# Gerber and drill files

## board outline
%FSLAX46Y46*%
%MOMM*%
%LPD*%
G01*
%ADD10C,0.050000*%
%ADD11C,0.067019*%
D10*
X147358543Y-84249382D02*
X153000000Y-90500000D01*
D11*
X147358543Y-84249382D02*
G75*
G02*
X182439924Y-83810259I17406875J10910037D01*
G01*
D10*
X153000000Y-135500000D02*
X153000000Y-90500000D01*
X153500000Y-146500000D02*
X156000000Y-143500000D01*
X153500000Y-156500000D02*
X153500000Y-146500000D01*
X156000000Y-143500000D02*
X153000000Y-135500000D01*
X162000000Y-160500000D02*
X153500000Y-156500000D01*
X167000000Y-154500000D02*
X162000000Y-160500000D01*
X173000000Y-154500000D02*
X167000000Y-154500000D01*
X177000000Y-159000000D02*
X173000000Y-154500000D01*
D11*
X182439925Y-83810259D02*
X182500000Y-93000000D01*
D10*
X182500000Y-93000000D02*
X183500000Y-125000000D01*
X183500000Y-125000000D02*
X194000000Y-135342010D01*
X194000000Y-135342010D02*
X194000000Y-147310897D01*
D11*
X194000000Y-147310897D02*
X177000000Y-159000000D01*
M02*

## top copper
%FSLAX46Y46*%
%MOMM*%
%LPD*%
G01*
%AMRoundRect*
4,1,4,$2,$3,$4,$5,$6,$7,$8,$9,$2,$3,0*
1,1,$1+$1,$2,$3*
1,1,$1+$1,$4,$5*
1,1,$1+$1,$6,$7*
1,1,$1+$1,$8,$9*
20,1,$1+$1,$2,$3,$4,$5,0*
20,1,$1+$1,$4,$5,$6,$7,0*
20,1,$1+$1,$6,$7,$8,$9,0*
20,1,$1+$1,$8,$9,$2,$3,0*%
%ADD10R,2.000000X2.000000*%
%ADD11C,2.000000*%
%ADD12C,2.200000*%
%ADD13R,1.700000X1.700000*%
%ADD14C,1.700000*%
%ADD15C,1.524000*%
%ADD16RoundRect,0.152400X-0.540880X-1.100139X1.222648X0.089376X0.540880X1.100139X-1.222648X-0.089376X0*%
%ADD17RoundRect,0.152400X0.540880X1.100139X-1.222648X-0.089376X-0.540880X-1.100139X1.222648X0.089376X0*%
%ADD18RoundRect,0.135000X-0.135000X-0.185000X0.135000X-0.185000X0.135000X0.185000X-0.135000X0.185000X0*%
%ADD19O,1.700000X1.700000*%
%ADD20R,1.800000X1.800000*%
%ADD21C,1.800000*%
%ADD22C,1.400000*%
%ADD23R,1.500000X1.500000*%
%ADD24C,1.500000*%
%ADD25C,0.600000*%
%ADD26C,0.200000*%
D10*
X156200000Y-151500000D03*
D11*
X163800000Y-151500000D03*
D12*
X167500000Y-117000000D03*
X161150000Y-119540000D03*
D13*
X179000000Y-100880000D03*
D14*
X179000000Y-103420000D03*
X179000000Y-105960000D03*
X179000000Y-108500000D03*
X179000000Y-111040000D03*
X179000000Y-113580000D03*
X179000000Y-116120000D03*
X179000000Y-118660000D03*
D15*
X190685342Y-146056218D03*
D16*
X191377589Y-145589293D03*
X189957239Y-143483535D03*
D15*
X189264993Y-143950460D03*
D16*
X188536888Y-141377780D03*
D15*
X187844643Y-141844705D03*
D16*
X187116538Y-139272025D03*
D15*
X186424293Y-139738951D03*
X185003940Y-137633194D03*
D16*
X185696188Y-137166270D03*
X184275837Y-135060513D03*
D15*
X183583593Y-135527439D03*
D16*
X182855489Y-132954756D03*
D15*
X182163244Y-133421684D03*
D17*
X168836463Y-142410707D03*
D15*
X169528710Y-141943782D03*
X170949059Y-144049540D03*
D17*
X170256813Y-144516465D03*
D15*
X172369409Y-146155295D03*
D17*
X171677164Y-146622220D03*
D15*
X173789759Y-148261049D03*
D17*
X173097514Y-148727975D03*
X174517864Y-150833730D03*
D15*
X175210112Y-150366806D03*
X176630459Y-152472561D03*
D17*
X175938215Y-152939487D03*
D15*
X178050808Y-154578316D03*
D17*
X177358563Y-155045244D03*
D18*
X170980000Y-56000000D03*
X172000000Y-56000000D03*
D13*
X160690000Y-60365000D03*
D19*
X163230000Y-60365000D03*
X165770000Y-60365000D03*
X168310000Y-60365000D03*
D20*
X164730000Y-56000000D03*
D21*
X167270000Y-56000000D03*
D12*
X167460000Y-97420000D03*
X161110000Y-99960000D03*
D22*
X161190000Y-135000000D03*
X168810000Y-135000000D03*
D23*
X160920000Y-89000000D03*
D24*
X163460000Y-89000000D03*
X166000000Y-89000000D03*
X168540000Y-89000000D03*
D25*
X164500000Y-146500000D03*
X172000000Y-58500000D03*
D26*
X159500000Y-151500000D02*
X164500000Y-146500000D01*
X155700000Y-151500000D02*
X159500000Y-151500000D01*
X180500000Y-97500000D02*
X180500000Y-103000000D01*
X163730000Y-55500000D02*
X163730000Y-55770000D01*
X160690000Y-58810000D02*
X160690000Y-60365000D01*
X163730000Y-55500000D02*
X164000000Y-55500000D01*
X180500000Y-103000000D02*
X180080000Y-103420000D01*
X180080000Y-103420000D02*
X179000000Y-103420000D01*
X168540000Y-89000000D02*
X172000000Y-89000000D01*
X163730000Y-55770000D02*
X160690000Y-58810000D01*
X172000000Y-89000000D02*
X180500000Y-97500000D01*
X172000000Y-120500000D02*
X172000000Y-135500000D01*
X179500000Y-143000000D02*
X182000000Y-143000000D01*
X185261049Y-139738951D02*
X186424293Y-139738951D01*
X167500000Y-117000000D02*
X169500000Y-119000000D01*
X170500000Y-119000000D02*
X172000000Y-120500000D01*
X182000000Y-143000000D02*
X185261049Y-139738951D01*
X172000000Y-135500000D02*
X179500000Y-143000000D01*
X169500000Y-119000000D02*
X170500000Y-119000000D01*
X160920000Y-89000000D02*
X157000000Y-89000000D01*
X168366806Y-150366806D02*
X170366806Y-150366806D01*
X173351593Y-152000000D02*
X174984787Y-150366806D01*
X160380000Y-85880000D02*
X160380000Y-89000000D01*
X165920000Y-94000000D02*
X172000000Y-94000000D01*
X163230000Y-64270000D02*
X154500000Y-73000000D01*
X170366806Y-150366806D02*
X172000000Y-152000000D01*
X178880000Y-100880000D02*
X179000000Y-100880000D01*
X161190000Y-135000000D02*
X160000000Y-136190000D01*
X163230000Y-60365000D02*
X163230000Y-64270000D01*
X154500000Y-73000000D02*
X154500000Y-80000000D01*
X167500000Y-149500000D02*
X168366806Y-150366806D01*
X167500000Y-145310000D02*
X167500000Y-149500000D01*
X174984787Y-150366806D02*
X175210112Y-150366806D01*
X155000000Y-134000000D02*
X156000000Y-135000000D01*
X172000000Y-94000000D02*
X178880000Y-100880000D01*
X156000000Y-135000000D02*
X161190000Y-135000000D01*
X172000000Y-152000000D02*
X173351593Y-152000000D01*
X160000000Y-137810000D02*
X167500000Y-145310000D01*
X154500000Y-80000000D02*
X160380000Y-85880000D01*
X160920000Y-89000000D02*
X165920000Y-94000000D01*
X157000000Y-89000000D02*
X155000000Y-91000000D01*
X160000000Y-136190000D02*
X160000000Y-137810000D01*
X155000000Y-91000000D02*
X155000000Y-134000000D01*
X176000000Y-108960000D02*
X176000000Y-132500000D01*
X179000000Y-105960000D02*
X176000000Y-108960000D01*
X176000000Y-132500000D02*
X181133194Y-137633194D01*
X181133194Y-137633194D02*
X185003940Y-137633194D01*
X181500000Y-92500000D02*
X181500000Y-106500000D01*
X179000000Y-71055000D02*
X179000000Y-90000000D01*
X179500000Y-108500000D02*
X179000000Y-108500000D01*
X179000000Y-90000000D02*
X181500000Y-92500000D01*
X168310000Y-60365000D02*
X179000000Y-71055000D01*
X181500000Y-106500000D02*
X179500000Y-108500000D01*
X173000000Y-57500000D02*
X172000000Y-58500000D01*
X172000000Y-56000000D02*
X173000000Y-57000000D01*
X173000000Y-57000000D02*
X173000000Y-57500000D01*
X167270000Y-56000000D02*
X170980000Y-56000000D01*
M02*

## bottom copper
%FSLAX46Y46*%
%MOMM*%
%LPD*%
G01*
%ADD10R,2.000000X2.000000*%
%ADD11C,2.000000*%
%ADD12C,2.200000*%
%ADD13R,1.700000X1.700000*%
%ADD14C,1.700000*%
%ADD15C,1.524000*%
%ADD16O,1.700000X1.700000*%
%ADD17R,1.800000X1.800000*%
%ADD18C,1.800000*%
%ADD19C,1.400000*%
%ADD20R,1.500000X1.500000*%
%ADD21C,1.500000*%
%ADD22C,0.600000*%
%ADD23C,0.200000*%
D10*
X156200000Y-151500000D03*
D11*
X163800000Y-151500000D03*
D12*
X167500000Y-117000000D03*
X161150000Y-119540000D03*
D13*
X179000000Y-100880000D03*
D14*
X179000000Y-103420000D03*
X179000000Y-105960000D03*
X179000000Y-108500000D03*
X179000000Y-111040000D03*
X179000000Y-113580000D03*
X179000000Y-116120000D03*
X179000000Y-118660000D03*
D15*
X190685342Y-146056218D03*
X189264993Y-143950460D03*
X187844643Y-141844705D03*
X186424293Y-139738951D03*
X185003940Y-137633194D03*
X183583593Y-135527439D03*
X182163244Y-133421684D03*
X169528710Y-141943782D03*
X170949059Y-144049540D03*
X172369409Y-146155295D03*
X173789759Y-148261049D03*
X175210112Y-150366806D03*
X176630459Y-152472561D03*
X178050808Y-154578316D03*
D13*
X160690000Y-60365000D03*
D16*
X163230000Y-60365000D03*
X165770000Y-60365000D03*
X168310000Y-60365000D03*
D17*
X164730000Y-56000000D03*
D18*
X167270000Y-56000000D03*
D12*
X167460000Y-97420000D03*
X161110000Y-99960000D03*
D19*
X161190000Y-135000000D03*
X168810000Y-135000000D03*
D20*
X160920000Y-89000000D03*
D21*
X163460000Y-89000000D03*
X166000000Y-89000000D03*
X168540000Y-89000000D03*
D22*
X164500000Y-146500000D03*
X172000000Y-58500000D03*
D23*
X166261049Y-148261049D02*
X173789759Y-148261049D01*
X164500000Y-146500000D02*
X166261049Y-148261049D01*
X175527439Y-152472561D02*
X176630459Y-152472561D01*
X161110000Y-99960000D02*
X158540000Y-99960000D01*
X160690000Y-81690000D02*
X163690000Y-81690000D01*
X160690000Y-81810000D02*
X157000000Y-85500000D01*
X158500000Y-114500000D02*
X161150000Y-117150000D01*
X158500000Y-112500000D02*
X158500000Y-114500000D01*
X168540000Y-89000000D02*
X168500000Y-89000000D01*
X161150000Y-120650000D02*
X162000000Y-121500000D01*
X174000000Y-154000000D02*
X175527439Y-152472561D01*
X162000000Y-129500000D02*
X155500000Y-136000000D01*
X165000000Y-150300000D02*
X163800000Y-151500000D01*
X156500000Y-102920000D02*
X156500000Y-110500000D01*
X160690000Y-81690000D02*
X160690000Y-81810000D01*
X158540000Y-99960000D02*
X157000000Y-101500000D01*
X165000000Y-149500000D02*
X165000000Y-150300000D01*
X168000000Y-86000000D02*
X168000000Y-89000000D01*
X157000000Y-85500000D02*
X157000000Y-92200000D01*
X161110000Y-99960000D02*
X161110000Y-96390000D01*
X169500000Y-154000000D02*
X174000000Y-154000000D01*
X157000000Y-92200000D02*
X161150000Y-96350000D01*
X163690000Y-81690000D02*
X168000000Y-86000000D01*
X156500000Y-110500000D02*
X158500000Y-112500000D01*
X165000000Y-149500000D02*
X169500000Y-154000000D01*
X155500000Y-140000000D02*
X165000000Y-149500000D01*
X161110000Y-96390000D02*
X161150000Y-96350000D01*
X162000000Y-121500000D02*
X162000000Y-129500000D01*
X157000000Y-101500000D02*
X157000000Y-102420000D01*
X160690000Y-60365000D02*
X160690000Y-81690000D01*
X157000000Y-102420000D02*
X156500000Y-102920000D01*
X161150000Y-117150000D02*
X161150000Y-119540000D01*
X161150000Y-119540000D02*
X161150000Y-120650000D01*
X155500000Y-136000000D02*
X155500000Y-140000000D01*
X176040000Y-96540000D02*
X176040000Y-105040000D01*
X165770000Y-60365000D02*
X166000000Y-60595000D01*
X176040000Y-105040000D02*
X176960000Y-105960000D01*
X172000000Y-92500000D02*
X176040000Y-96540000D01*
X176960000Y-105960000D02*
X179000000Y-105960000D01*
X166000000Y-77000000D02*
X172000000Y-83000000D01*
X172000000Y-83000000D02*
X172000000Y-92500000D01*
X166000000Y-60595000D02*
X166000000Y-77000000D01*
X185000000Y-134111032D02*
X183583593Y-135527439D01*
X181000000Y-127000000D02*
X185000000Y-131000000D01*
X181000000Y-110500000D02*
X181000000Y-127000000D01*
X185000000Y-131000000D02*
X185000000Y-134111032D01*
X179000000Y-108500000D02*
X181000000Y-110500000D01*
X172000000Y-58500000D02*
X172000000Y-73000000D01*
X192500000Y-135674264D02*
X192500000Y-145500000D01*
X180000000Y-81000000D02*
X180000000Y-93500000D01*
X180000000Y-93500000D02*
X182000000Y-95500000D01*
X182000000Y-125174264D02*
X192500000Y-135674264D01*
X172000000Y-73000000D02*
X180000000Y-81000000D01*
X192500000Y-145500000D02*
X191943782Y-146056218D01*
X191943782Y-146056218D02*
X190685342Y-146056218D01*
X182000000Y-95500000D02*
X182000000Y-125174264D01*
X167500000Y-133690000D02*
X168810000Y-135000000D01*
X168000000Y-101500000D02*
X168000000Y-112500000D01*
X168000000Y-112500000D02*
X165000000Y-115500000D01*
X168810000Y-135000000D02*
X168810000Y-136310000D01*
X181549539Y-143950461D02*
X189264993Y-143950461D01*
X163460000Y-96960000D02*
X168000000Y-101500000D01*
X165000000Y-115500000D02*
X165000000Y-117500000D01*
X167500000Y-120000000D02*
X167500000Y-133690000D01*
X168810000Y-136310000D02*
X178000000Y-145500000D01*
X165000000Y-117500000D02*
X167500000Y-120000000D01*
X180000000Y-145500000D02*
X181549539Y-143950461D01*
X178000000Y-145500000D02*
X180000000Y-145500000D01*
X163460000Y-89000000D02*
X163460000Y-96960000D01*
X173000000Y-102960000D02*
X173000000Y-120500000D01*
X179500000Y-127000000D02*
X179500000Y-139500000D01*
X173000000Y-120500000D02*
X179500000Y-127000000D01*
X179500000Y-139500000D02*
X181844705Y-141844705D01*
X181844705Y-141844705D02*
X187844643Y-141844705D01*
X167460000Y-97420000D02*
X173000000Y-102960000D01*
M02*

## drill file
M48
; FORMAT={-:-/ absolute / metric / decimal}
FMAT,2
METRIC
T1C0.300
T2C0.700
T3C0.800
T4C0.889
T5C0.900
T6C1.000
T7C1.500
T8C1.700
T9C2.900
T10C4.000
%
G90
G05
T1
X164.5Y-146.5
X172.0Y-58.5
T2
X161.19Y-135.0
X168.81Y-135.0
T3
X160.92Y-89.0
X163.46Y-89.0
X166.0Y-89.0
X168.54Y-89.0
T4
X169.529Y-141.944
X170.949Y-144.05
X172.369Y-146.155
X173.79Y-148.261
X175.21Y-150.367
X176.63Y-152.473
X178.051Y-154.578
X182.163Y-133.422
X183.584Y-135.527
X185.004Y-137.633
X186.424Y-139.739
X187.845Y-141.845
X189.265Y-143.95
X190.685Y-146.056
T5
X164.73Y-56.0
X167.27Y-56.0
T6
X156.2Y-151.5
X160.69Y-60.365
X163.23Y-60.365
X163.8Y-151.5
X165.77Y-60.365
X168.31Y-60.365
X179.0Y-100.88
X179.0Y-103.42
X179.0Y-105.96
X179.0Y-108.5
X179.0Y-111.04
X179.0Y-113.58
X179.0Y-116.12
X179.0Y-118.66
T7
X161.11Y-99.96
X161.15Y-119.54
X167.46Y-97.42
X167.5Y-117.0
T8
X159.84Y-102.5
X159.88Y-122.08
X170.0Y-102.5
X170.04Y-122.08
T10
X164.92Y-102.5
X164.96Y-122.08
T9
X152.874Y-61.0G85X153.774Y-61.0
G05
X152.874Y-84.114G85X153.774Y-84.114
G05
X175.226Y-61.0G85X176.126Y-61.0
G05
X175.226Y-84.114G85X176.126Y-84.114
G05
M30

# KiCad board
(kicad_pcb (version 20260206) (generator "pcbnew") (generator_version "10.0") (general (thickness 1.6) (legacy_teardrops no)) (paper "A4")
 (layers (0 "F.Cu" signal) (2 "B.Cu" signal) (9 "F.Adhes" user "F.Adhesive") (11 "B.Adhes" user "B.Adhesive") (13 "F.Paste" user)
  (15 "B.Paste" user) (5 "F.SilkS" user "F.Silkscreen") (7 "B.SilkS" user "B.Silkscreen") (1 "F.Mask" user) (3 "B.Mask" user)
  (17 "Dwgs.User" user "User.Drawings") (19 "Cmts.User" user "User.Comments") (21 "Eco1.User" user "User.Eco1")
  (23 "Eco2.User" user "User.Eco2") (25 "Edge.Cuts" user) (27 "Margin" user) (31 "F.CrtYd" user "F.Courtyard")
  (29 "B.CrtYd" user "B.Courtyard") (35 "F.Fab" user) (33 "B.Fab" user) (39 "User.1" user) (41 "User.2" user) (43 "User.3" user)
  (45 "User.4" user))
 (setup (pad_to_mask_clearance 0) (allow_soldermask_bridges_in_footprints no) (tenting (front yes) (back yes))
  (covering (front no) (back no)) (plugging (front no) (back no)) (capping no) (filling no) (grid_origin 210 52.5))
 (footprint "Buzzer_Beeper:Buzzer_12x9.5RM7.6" (layer "F.Cu") (at 156.2 151.5)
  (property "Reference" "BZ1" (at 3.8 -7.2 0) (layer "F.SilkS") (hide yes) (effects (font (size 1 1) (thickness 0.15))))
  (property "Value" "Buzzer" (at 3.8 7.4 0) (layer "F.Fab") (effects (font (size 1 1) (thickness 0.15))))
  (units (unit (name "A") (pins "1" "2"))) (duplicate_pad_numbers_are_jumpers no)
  (pad "1" thru_hole rect (at 0 0) (size 2 2) (drill 1) (layers "*.Cu" "*.Mask") (remove_unused_layers no) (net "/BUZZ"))
  (pad "2" thru_hole circle (at 7.6 0) (size 2 2) (drill 1) (layers "*.Cu" "*.Mask") (remove_unused_layers no) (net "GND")))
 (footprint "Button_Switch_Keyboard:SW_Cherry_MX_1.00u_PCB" (layer "F.Cu") (at 167.5 117)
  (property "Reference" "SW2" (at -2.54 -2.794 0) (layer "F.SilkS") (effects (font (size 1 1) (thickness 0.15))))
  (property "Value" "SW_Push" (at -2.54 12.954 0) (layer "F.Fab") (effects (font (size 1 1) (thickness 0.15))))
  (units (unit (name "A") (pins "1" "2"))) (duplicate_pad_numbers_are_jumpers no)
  (pad "" np_thru_hole circle (at -7.62 5.08) (size 1.7 1.7) (drill 1.7) (layers "*.Cu" "*.Mask"))
  (pad "" np_thru_hole circle (at -2.54 5.08) (size 4 4) (drill 4) (layers "*.Cu" "*.Mask"))
  (pad "" np_thru_hole circle (at 2.54 5.08) (size 1.7 1.7) (drill 1.7) (layers "*.Cu" "*.Mask"))
  (pad "1" thru_hole circle (at 0 0) (size 2.2 2.2) (drill 1.5) (layers "*.Cu" "*.Mask") (remove_unused_layers no) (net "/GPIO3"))
  (pad "2" thru_hole circle (at -6.35 2.54) (size 2.2 2.2) (drill 1.5) (layers "*.Cu" "*.Mask") (remove_unused_layers no) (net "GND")))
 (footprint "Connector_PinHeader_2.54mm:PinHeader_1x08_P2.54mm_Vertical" (layer "F.Cu") (at 179 100.88)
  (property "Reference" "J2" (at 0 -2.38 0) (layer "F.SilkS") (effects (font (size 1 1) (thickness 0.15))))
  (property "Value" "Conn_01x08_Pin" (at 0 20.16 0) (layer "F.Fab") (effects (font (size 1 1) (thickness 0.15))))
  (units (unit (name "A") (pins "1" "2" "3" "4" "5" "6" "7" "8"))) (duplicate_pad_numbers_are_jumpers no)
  (pad "1" thru_hole rect (at 0 0) (size 1.7 1.7) (drill 1) (layers "*.Cu" "*.Mask") (remove_unused_layers no) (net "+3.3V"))
  (pad "2" thru_hole circle (at 0 2.54) (size 1.7 1.7) (drill 1) (layers "*.Cu" "*.Mask") (remove_unused_layers no) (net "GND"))
  (pad "3" thru_hole circle (at 0 5.08) (size 1.7 1.7) (drill 1) (layers "*.Cu" "*.Mask") (remove_unused_layers no) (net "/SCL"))
  (pad "4" thru_hole circle (at 0 7.62) (size 1.7 1.7) (drill 1) (layers "*.Cu" "*.Mask") (remove_unused_layers no) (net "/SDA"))
  (pad "5" thru_hole circle (at 0 10.16) (size 1.7 1.7) (drill 1) (layers "*.Cu" "*.Mask") (remove_unused_layers no)
   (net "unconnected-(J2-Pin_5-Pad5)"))
  (pad "6" thru_hole circle (at 0 12.7) (size 1.7 1.7) (drill 1) (layers "*.Cu" "*.Mask") (remove_unused_layers no)
   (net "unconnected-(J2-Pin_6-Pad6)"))
  (pad "7" thru_hole circle (at 0 15.24) (size 1.7 1.7) (drill 1) (layers "*.Cu" "*.Mask") (remove_unused_layers no)
   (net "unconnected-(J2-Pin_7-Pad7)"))
  (pad "8" thru_hole circle (at 0 17.78) (size 1.7 1.7) (drill 1) (layers "*.Cu" "*.Mask") (remove_unused_layers no)
   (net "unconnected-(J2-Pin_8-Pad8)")))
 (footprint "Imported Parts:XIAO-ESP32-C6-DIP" (layer "F.Cu") (at 180.107026 144 -56)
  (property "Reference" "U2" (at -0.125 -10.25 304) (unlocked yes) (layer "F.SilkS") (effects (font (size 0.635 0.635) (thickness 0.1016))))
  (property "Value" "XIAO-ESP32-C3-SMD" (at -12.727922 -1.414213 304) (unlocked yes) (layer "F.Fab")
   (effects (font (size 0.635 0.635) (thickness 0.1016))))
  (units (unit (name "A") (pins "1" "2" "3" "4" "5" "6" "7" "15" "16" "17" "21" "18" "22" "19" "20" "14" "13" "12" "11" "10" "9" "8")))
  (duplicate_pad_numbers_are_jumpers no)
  (pad "1" thru_hole circle (at 7.620001 -7.619999 34) (size 1.524 1.524) (drill 0.889) (layers "*.Cu" "*.Mask") (remove_unused_layers no)
   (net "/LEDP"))
  (pad "1" smd roundrect (at 7.620002 -8.454999 34) (size 2.432 1.524) (layers "F.Cu" "F.Mask") (roundrect_rratio 0.1) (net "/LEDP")
   (thermal_bridge_angle 45))
  (pad "2" smd roundrect (at 5.08 -8.455 34) (size 2.432 1.524) (layers "F.Cu" "F.Mask") (roundrect_rratio 0.1) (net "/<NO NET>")
   (thermal_bridge_angle 45))
  (pad "2" thru_hole circle (at 5.08 -7.620001 34) (size 1.524 1.524) (drill 0.889) (layers "*.Cu" "*.Mask") (remove_unused_layers no)
   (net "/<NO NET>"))
  (pad "3" smd roundrect (at 2.54 -8.454999 34) (size 2.432 1.524) (layers "F.Cu" "F.Mask") (roundrect_rratio 0.1) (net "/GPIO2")
   (thermal_bridge_angle 45))
  (pad "3" thru_hole circle (at 2.54 -7.620001 34) (size 1.524 1.524) (drill 0.889) (layers "*.Cu" "*.Mask") (remove_unused_layers no)
   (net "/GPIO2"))
  (pad "4" smd roundrect (at 0 -8.454999 34) (size 2.432 1.524) (layers "F.Cu" "F.Mask") (roundrect_rratio 0.1) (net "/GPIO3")
   (thermal_bridge_angle 45))
  (pad "4" thru_hole circle (at 0.000001 -7.62 34) (size 1.524 1.524) (drill 0.889) (layers "*.Cu" "*.Mask") (remove_unused_layers no)
   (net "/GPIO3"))
  (pad "5" thru_hole circle (at -2.540002 -7.619998 34) (size 1.524 1.524) (drill 0.889) (layers "*.Cu" "*.Mask") (remove_unused_layers no)
   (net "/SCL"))
  (pad "5" smd roundrect (at -2.539999 -8.454999 34) (size 2.432 1.524) (layers "F.Cu" "F.Mask") (roundrect_rratio 0.1) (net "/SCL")
   (thermal_bridge_angle 45))
  (pad "6" smd roundrect (at -5.080001 -8.454999 34) (size 2.432 1.524) (layers "F.Cu" "F.Mask") (roundrect_rratio 0.1) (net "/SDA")
   (thermal_bridge_angle 45))
  (pad "6" thru_hole circle (at -5.08 -7.620001 34) (size 1.524 1.524) (drill 0.889) (layers "*.Cu" "*.Mask") (remove_unused_layers no)
   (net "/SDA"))
  (pad "7" smd roundrect (at -7.620001 -8.455001 34) (size 2.432 1.524) (layers "F.Cu" "F.Mask") (roundrect_rratio 0.1)
   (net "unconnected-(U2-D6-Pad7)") (thermal_bridge_angle 45))
  (pad "7" thru_hole circle (at -7.619999 -7.620001 34) (size 1.524 1.524) (drill 0.889) (layers "*.Cu" "*.Mask") (remove_unused_layers no)
   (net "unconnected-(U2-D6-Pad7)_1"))
  (pad "8" smd roundrect (at -7.620002 8.454999 214) (size 2.432 1.524) (layers "F.Cu" "F.Mask") (roundrect_rratio 0.1)
   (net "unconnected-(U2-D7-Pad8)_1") (thermal_bridge_angle 45))
  (pad "8" thru_hole circle (at -7.620001 7.619999 214) (size 1.524 1.524) (drill 0.889) (layers "*.Cu" "*.Mask") (remove_unused_layers no)
   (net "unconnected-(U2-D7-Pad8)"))
  (pad "9" thru_hole circle (at -5.08 7.620001 214) (size 1.524 1.524) (drill 0.889) (layers "*.Cu" "*.Mask") (remove_unused_layers no)
   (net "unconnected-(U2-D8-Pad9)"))
  (pad "9" smd roundrect (at -5.08 8.455 214) (size 2.432 1.524) (layers "F.Cu" "F.Mask") (roundrect_rratio 0.1)
   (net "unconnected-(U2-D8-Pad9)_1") (thermal_bridge_angle 45))
  (pad "10" thru_hole circle (at -2.54 7.620001 214) (size 1.524 1.524) (drill 0.889) (layers "*.Cu" "*.Mask") (remove_unused_layers no)
   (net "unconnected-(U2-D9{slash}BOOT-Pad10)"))
  (pad "10" smd roundrect (at -2.54 8.454999 214) (size 2.432 1.524) (layers "F.Cu" "F.Mask") (roundrect_rratio 0.1)
   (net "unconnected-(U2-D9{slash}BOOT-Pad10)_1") (thermal_bridge_angle 45))
  (pad "11" thru_hole circle (at -0.000001 7.62 214) (size 1.524 1.524) (drill 0.889) (layers "*.Cu" "*.Mask") (remove_unused_layers no)
   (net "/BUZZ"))
  (pad "11" smd roundrect (at 0 8.454999 214) (size 2.432 1.524) (layers "F.Cu" "F.Mask") (roundrect_rratio 0.1) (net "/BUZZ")
   (thermal_bridge_angle 45))
  (pad "12" smd roundrect (at 2.539999 8.454999 214) (size 2.432 1.524) (layers "F.Cu" "F.Mask") (roundrect_rratio 0.1) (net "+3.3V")
   (thermal_bridge_angle 45))
  (pad "12" thru_hole circle (at 2.540002 7.619998 214) (size 1.524 1.524) (drill 0.889) (layers "*.Cu" "*.Mask") (remove_unused_layers no)
   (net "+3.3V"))
  (pad "13" thru_hole circle (at 5.08 7.620001 214) (size 1.524 1.524) (drill 0.889) (layers "*.Cu" "*.Mask") (remove_unused_layers no)
   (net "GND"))
  (pad "13" smd roundrect (at 5.080001 8.454999 214) (size 2.432 1.524) (layers "F.Cu" "F.Mask") (roundrect_rratio 0.1) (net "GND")
   (thermal_bridge_angle 45))
  (pad "14" thru_hole circle (at 7.619999 7.620001 214) (size 1.524 1.524) (drill 0.889) (layers "*.Cu" "*.Mask") (remove_unused_layers no)
   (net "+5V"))
  (pad "14" smd roundrect (at 7.620001 8.455001 214) (size 2.432 1.524) (layers "F.Cu" "F.Mask") (roundrect_rratio 0.1) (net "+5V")
   (thermal_bridge_angle 45)))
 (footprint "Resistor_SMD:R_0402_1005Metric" (layer "F.Cu") (at 171.49 56)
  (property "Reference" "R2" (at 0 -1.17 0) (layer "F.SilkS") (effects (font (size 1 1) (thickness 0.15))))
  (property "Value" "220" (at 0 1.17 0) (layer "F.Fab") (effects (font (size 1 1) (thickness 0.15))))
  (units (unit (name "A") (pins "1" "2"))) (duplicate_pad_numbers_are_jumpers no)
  (pad "1" smd roundrect (at -0.51 0) (size 0.54 0.64) (layers "F.Cu" "F.Mask" "F.Paste") (roundrect_rratio 0.25) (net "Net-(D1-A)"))
  (pad "2" smd roundrect (at 0.51 0) (size 0.54 0.64) (layers "F.Cu" "F.Mask" "F.Paste") (roundrect_rratio 0.25) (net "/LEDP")))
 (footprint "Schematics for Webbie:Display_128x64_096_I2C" (layer "F.Cu") (at 164.5 60.365)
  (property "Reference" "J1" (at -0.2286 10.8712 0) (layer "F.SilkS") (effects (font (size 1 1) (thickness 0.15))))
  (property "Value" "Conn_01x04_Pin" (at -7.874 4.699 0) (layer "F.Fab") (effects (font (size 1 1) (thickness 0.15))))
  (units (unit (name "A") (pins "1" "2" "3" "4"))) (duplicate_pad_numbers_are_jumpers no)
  (pad "" np_thru_hole oval (at -11.176 0.635) (size 3.8 2.9) (drill oval 3.8 2.9) (layers "*.Cu" "*.Mask"))
  (pad "" np_thru_hole oval (at -11.176 23.749) (size 3.8 2.9) (drill oval 3.8 2.9) (layers "*.Cu" "*.Mask"))
  (pad "" np_thru_hole oval (at 11.176 0.635) (size 3.8 2.9) (drill oval 3.8 2.9) (layers "*.Cu" "*.Mask"))
  (pad "" np_thru_hole oval (at 11.176 23.749) (size 3.8 2.9) (drill oval 3.8 2.9) (layers "*.Cu" "*.Mask"))
  (pad "1" thru_hole rect (at -3.81 0 90) (size 1.7 1.7) (drill 1) (layers "*.Cu" "*.Mask") (remove_unused_layers no) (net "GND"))
  (pad "2" thru_hole oval (at -1.27 0 90) (size 1.7 1.7) (drill 1) (layers "*.Cu" "*.Mask") (remove_unused_layers no) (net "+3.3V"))
  (pad "3" thru_hole oval (at 1.27 0 90) (size 1.7 1.7) (drill 1) (layers "*.Cu" "*.Mask") (remove_unused_layers no) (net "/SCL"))
  (pad "4" thru_hole oval (at 3.81 0 90) (size 1.7 1.7) (drill 1) (layers "*.Cu" "*.Mask") (remove_unused_layers no) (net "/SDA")))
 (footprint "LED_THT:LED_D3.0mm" (layer "F.Cu") (at 164.73 56)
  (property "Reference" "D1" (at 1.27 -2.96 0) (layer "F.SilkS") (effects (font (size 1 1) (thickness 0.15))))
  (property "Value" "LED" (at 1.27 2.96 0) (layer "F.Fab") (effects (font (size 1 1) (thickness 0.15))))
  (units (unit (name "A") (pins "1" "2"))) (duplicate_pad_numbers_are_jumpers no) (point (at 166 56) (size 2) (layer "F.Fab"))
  (pad "1" thru_hole rect (at 0 0) (size 1.8 1.8) (drill 0.9) (layers "*.Cu" "*.Mask") (remove_unused_layers no) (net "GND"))
  (pad "2" thru_hole circle (at 2.54 0) (size 1.8 1.8) (drill 0.9) (layers "*.Cu" "*.Mask") (remove_unused_layers no) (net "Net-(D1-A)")))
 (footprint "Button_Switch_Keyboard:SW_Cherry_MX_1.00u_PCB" (layer "F.Cu") (at 167.46 97.42)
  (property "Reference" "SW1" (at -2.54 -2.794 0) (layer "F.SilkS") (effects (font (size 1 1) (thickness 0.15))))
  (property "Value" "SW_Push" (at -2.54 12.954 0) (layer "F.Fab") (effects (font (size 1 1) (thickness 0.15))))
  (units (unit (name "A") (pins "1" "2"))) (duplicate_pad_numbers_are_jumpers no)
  (pad "" np_thru_hole circle (at -7.62 5.08) (size 1.7 1.7) (drill 1.7) (layers "*.Cu" "*.Mask"))
  (pad "" np_thru_hole circle (at -2.54 5.08) (size 4 4) (drill 4) (layers "*.Cu" "*.Mask"))
  (pad "" np_thru_hole circle (at 2.54 5.08) (size 1.7 1.7) (drill 1.7) (layers "*.Cu" "*.Mask"))
  (pad "1" thru_hole circle (at 0 0) (size 2.2 2.2) (drill 1.5) (layers "*.Cu" "*.Mask") (remove_unused_layers no) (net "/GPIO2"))
  (pad "2" thru_hole circle (at -6.35 2.54) (size 2.2 2.2) (drill 1.5) (layers "*.Cu" "*.Mask") (remove_unused_layers no) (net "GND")))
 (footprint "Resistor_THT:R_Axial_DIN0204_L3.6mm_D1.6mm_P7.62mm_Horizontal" (layer "F.Cu") (at 161.19 135)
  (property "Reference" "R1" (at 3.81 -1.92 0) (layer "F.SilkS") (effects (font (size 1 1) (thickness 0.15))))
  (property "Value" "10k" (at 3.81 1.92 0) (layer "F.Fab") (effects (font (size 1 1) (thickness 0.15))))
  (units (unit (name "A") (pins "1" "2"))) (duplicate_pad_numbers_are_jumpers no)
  (pad "1" thru_hole circle (at 0 0) (size 1.4 1.4) (drill 0.7) (layers "*.Cu" "*.Mask") (remove_unused_layers no) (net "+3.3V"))
  (pad "2" thru_hole circle (at 7.62 0) (size 1.4 1.4) (drill 0.7) (layers "*.Cu" "*.Mask") (remove_unused_layers no) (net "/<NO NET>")))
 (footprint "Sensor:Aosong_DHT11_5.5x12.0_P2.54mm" (layer "F.Cu") (at 160.92 89 90)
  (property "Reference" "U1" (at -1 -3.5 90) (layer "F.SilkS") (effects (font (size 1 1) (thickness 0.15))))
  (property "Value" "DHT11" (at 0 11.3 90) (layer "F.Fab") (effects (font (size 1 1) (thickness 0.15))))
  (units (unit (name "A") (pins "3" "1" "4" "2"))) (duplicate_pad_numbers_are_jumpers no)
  (pad "1" thru_hole rect (at 0 0 90) (size 1.5 1.5) (drill 0.8) (layers "*.Cu" "*.Mask") (remove_unused_layers no) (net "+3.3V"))
  (pad "2" thru_hole circle (at 0 2.54 90) (size 1.5 1.5) (drill 0.8) (layers "*.Cu" "*.Mask") (remove_unused_layers no) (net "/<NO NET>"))
  (pad "3" thru_hole circle (at 0 5.08 90) (size 1.5 1.5) (drill 0.8) (layers "*.Cu" "*.Mask") (remove_unused_layers no)
   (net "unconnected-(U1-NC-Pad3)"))
  (pad "4" thru_hole circle (at 0 7.62 90) (size 1.5 1.5) (drill 0.8) (layers "*.Cu" "*.Mask") (remove_unused_layers no) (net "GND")))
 (gr_line (start 147.358543 84.249382) (end 153 90.5) (stroke (width 0.05) (type default)) (layer "Edge.Cuts"))
 (gr_arc (start 147.358543 84.249382) (mid 164.508292 52.797628) (end 182.439925 83.810259) (stroke (width 0.067019) (type default))
  (layer "Edge.Cuts"))
 (gr_line (start 153 135.5) (end 153 90.5) (stroke (width 0.05) (type default)) (layer "Edge.Cuts"))
 (gr_line (start 153.5 146.5) (end 156 143.5) (stroke (width 0.05) (type default)) (layer "Edge.Cuts"))
 (gr_line (start 153.5 156.5) (end 153.5 146.5) (stroke (width 0.05) (type default)) (layer "Edge.Cuts"))
 (gr_line (start 156 143.5) (end 153 135.5) (stroke (width 0.05) (type default)) (layer "Edge.Cuts"))
 (gr_line (start 162 160.5) (end 153.5 156.5) (stroke (width 0.05) (type default)) (layer "Edge.Cuts"))
 (gr_line (start 167 154.5) (end 162 160.5) (stroke (width 0.05) (type default)) (layer "Edge.Cuts"))
 (gr_line (start 173 154.5) (end 167 154.5) (stroke (width 0.05) (type default)) (layer "Edge.Cuts"))
 (gr_line (start 177 159) (end 173 154.5) (stroke (width 0.05) (type default)) (layer "Edge.Cuts"))
 (gr_line (start 182.439925 83.810259) (end 182.5 93) (stroke (width 0.067019) (type default)) (layer "Edge.Cuts"))
 (gr_line (start 182.5 93) (end 183.5 125) (stroke (width 0.05) (type default)) (layer "Edge.Cuts"))
 (gr_line (start 183.5 125) (end 194 135.34201) (stroke (width 0.05) (type default)) (layer "Edge.Cuts"))
 (gr_line (start 194 135.34201) (end 194 147.310897) (stroke (width 0.05) (type default)) (layer "Edge.Cuts"))
 (gr_line (start 194 147.310897) (end 177 159) (stroke (width 0.067019) (type default)) (layer "Edge.Cuts"))
 (segment (start 159.5 151.5) (end 164.5 146.5) (width 0.2) (layer "F.Cu") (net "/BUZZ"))
 (segment (start 155.7 151.5) (end 159.5 151.5) (width 0.2) (layer "F.Cu") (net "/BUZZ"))
 (via (at 164.5 146.5) (size 0.6) (drill 0.3) (layers "F.Cu" "B.Cu") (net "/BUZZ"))
 (segment (start 166.261049 148.261049) (end 173.789759 148.261049) (width 0.2) (layer "B.Cu") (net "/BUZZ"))
 (segment (start 164.5 146.5) (end 166.261049 148.261049) (width 0.2) (layer "B.Cu") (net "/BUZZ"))
 (segment (start 180.5 97.5) (end 180.5 103) (width 0.2) (layer "F.Cu") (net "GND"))
 (segment (start 163.73 55.5) (end 163.73 55.77) (width 0.2) (layer "F.Cu") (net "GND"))
 (segment (start 160.69 58.81) (end 160.69 60.365) (width 0.2) (layer "F.Cu") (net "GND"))
 (segment (start 163.73 55.5) (end 164 55.5) (width 0.2) (layer "F.Cu") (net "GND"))
 (segment (start 180.5 103) (end 180.08 103.42) (width 0.2) (layer "F.Cu") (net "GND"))
 (segment (start 180.08 103.42) (end 179 103.42) (width 0.2) (layer "F.Cu") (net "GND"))
 (segment (start 168.54 89) (end 172 89) (width 0.2) (layer "F.Cu") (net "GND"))
 (segment (start 163.73 55.77) (end 160.69 58.81) (width 0.2) (layer "F.Cu") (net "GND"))
 (segment (start 172 89) (end 180.5 97.5) (width 0.2) (layer "F.Cu") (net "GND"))
 (segment (start 175.527439 152.472561) (end 176.630459 152.472561) (width 0.2) (layer "B.Cu") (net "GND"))
 (segment (start 161.11 99.96) (end 158.54 99.96) (width 0.2) (layer "B.Cu") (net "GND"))
 (segment (start 160.69 81.69) (end 163.69 81.69) (width 0.2) (layer "B.Cu") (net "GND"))
 (segment (start 160.69 81.81) (end 157 85.5) (width 0.2) (layer "B.Cu") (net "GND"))
 (segment (start 158.5 114.5) (end 161.15 117.15) (width 0.2) (layer "B.Cu") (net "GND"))
 (segment (start 158.5 112.5) (end 158.5 114.5) (width 0.2) (layer "B.Cu") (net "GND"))
 (segment (start 168.54 89) (end 168.5 89) (width 0.2) (layer "B.Cu") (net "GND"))
 (segment (start 161.15 120.65) (end 162 121.5) (width 0.2) (layer "B.Cu") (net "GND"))
 (segment (start 174 154) (end 175.527439 152.472561) (width 0.2) (layer "B.Cu") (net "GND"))
 (segment (start 162 129.5) (end 155.5 136) (width 0.2) (layer "B.Cu") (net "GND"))
 (segment (start 165 150.3) (end 163.8 151.5) (width 0.2) (layer "B.Cu") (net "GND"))
 (segment (start 156.5 102.92) (end 156.5 110.5) (width 0.2) (layer "B.Cu") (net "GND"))
 (segment (start 160.69 81.69) (end 160.69 81.81) (width 0.2) (layer "B.Cu") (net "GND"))
 (segment (start 158.54 99.96) (end 157 101.5) (width 0.2) (layer "B.Cu") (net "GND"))
 (segment (start 165 149.5) (end 165 150.3) (width 0.2) (layer "B.Cu") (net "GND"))
 (segment (start 168 86) (end 168 89) (width 0.2) (layer "B.Cu") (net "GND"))
 (segment (start 157 85.5) (end 157 92.2) (width 0.2) (layer "B.Cu") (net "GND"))
 (segment (start 161.11 99.96) (end 161.11 96.39) (width 0.2) (layer "B.Cu") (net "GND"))
 (segment (start 169.5 154) (end 174 154) (width 0.2) (layer "B.Cu") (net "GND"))
 (segment (start 157 92.2) (end 161.15 96.35) (width 0.2) (layer "B.Cu") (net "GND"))
 (segment (start 163.69 81.69) (end 168 86) (width 0.2) (layer "B.Cu") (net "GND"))
 (segment (start 156.5 110.5) (end 158.5 112.5) (width 0.2) (layer "B.Cu") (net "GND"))
 (segment (start 165 149.5) (end 169.5 154) (width 0.2) (layer "B.Cu") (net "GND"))
 (segment (start 155.5 140) (end 165 149.5) (width 0.2) (layer "B.Cu") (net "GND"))
 (segment (start 161.11 96.39) (end 161.15 96.35) (width 0.2) (layer "B.Cu") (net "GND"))
 (segment (start 162 121.5) (end 162 129.5) (width 0.2) (layer "B.Cu") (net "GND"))
 (segment (start 157 101.5) (end 157 102.42) (width 0.2) (layer "B.Cu") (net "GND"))
 (segment (start 160.69 60.365) (end 160.69 81.69) (width 0.2) (layer "B.Cu") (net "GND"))
 (segment (start 157 102.42) (end 156.5 102.92) (width 0.2) (layer "B.Cu") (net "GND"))
 (segment (start 161.15 117.15) (end 161.15 119.54) (width 0.2) (layer "B.Cu") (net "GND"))
 (segment (start 161.15 119.54) (end 161.15 120.65) (width 0.2) (layer "B.Cu") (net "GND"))
 (segment (start 155.5 136) (end 155.5 140) (width 0.2) (layer "B.Cu") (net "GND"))
 (segment (start 172 120.5) (end 172 135.5) (width 0.2) (layer "F.Cu") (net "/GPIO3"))
 (segment (start 179.5 143) (end 182 143) (width 0.2) (layer "F.Cu") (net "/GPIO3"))
 (segment (start 185.261049 139.738951) (end 186.424293 139.738951) (width 0.2) (layer "F.Cu") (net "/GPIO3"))
 (segment (start 167.5 117) (end 169.5 119) (width 0.2) (layer "F.Cu") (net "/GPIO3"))
 (segment (start 170.5 119) (end 172 120.5) (width 0.2) (layer "F.Cu") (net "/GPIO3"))
 (segment (start 182 143) (end 185.261049 139.738951) (width 0.2) (layer "F.Cu") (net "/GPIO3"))
 (segment (start 172 135.5) (end 179.5 143) (width 0.2) (layer "F.Cu") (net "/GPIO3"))
 (segment (start 169.5 119) (end 170.5 119) (width 0.2) (layer "F.Cu") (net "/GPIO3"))
 (segment (start 160.92 89) (end 157 89) (width 0.2) (layer "F.Cu") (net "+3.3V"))
 (segment (start 168.366806 150.366806) (end 170.366806 150.366806) (width 0.2) (layer "F.Cu") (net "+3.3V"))
 (segment (start 173.351593 152) (end 174.984787 150.366806) (width 0.2) (layer "F.Cu") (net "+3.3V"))
 (segment (start 160.38 85.88) (end 160.38 89) (width 0.2) (layer "F.Cu") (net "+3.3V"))
 (segment (start 165.92 94) (end 172 94) (width 0.2) (layer "F.Cu") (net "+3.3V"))
 (segment (start 163.23 64.27) (end 154.5 73) (width 0.2) (layer "F.Cu") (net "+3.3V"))
 (segment (start 170.366806 150.366806) (end 172 152) (width 0.2) (layer "F.Cu") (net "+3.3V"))
 (segment (start 178.88 100.88) (end 179 100.88) (width 0.2) (layer "F.Cu") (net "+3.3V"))
 (segment (start 161.19 135) (end 160 136.19) (width 0.2) (layer "F.Cu") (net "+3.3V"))
 (segment (start 163.23 60.365) (end 163.23 64.27) (width 0.2) (layer "F.Cu") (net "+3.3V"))
 (segment (start 154.5 73) (end 154.5 80) (width 0.2) (layer "F.Cu") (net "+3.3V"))
 (segment (start 167.5 149.5) (end 168.366806 150.366806) (width 0.2) (layer "F.Cu") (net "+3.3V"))
 (segment (start 167.5 145.31) (end 167.5 149.5) (width 0.2) (layer "F.Cu") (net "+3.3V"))
 (segment (start 174.984787 150.366806) (end 175.210112 150.366806) (width 0.2) (layer "F.Cu") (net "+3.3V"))
 (segment (start 155 134) (end 156 135) (width 0.2) (layer "F.Cu") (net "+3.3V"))
 (segment (start 172 94) (end 178.88 100.88) (width 0.2) (layer "F.Cu") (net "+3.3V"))
 (segment (start 156 135) (end 161.19 135) (width 0.2) (layer "F.Cu") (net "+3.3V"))
 (segment (start 172 152) (end 173.351593 152) (width 0.2) (layer "F.Cu") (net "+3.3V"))
 (segment (start 160 137.81) (end 167.5 145.31) (width 0.2) (layer "F.Cu") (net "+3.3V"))
 (segment (start 154.5 80) (end 160.38 85.88) (width 0.2) (layer "F.Cu") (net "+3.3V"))
 (segment (start 160.92 89) (end 165.92 94) (width 0.2) (layer "F.Cu") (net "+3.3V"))
 (segment (start 157 89) (end 155 91) (width 0.2) (layer "F.Cu") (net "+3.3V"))
 (segment (start 160 136.19) (end 160 137.81) (width 0.2) (layer "F.Cu") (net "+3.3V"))
 (segment (start 155 91) (end 155 134) (width 0.2) (layer "F.Cu") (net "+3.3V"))
 (segment (start 176 108.96) (end 176 132.5) (width 0.2) (layer "F.Cu") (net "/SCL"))
 (segment (start 179 105.96) (end 176 108.96) (width 0.2) (layer "F.Cu") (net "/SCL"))
 (segment (start 176 132.5) (end 181.133194 137.633194) (width 0.2) (layer "F.Cu") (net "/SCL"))
 (segment (start 181.133194 137.633194) (end 185.00394 137.633194) (width 0.2) (layer "F.Cu") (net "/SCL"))
 (segment (start 176.04 96.54) (end 176.04 105.04) (width 0.2) (layer "B.Cu") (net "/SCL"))
 (segment (start 165.77 60.365) (end 166 60.595) (width 0.2) (layer "B.Cu") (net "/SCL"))
 (segment (start 176.04 105.04) (end 176.96 105.96) (width 0.2) (layer "B.Cu") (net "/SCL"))
 (segment (start 172 92.5) (end 176.04 96.54) (width 0.2) (layer "B.Cu") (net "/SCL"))
 (segment (start 176.96 105.96) (end 179 105.96) (width 0.2) (layer "B.Cu") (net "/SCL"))
 (segment (start 166 77) (end 172 83) (width 0.2) (layer "B.Cu") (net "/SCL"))
 (segment (start 172 83) (end 172 92.5) (width 0.2) (layer "B.Cu") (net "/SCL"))
 (segment (start 166 60.595) (end 166 77) (width 0.2) (layer "B.Cu") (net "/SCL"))
 (segment (start 181.5 92.5) (end 181.5 106.5) (width 0.2) (layer "F.Cu") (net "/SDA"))
 (segment (start 179 71.055) (end 179 90) (width 0.2) (layer "F.Cu") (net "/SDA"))
 (segment (start 179.5 108.5) (end 179 108.5) (width 0.2) (layer "F.Cu") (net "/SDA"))
 (segment (start 179 90) (end 181.5 92.5) (width 0.2) (layer "F.Cu") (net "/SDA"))
 (segment (start 168.31 60.365) (end 179 71.055) (width 0.2) (layer "F.Cu") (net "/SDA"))
 (segment (start 181.5 106.5) (end 179.5 108.5) (width 0.2) (layer "F.Cu") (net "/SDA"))
 (segment (start 185 134.111032) (end 183.583593 135.527439) (width 0.2) (layer "B.Cu") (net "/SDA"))
 (segment (start 181 127) (end 185 131) (width 0.2) (layer "B.Cu") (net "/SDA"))
 (segment (start 181 110.5) (end 181 127) (width 0.2) (layer "B.Cu") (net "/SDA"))
 (segment (start 185 131) (end 185 134.111032) (width 0.2) (layer "B.Cu") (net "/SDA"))
 (segment (start 179 108.5) (end 181 110.5) (width 0.2) (layer "B.Cu") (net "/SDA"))
 (segment (start 173 57.5) (end 172 58.5) (width 0.2) (layer "F.Cu") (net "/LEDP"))
 (segment (start 172 56) (end 173 57) (width 0.2) (layer "F.Cu") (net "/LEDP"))
 (segment (start 173 57) (end 173 57.5) (width 0.2) (layer "F.Cu") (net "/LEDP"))
 (via (at 172 58.5) (size 0.6) (drill 0.3) (layers "F.Cu" "B.Cu") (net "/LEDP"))
 (segment (start 172 58.5) (end 172 73) (width 0.2) (layer "B.Cu") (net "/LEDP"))
 (segment (start 192.5 135.674264) (end 192.5 145.5) (width 0.2) (layer "B.Cu") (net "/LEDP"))
 (segment (start 180 81) (end 180 93.5) (width 0.2) (layer "B.Cu") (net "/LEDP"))
 (segment (start 180 93.5) (end 182 95.5) (width 0.2) (layer "B.Cu") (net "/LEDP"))
 (segment (start 182 125.174264) (end 192.5 135.674264) (width 0.2) (layer "B.Cu") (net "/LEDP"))
 (segment (start 172 73) (end 180 81) (width 0.2) (layer "B.Cu") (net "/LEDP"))
 (segment (start 192.5 145.5) (end 191.943782 146.056218) (width 0.2) (layer "B.Cu") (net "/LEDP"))
 (segment (start 191.943782 146.056218) (end 190.685342 146.056218) (width 0.2) (layer "B.Cu") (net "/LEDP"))
 (segment (start 182 95.5) (end 182 125.174264) (width 0.2) (layer "B.Cu") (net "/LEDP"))
 (segment (start 167.5 133.69) (end 168.81 135) (width 0.2) (layer "B.Cu") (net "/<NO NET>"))
 (segment (start 168 101.5) (end 168 112.5) (width 0.2) (layer "B.Cu") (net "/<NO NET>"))
 (segment (start 168 112.5) (end 165 115.5) (width 0.2) (layer "B.Cu") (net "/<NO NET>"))
 (segment (start 168.81 135) (end 168.81 136.31) (width 0.2) (layer "B.Cu") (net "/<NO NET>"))
 (segment (start 181.549539 143.950461) (end 189.264993 143.950461) (width 0.2) (layer "B.Cu") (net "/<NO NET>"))
 (segment (start 163.46 96.96) (end 168 101.5) (width 0.2) (layer "B.Cu") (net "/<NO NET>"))
 (segment (start 165 115.5) (end 165 117.5) (width 0.2) (layer "B.Cu") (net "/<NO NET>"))
 (segment (start 167.5 120) (end 167.5 133.69) (width 0.2) (layer "B.Cu") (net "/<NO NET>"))
 (segment (start 168.81 136.31) (end 178 145.5) (width 0.2) (layer "B.Cu") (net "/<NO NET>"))
 (segment (start 165 117.5) (end 167.5 120) (width 0.2) (layer "B.Cu") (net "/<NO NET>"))
 (segment (start 180 145.5) (end 181.549539 143.950461) (width 0.2) (layer "B.Cu") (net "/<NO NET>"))
 (segment (start 178 145.5) (end 180 145.5) (width 0.2) (layer "B.Cu") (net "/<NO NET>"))
 (segment (start 163.46 89) (end 163.46 96.96) (width 0.2) (layer "B.Cu") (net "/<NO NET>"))
 (segment (start 173 102.96) (end 173 120.5) (width 0.2) (layer "B.Cu") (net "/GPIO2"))
 (segment (start 179.5 127) (end 179.5 139.5) (width 0.2) (layer "B.Cu") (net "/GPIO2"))
 (segment (start 173 120.5) (end 179.5 127) (width 0.2) (layer "B.Cu") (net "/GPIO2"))
 (segment (start 179.5 139.5) (end 181.844705 141.844705) (width 0.2) (layer "B.Cu") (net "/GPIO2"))
 (segment (start 181.844705 141.844705) (end 187.844643 141.844705) (width 0.2) (layer "B.Cu") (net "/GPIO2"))
 (segment (start 167.46 97.42) (end 173 102.96) (width 0.2) (layer "B.Cu") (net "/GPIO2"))
 (segment (start 167.27 56) (end 170.98 56) (width 0.2) (layer "F.Cu") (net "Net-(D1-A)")))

